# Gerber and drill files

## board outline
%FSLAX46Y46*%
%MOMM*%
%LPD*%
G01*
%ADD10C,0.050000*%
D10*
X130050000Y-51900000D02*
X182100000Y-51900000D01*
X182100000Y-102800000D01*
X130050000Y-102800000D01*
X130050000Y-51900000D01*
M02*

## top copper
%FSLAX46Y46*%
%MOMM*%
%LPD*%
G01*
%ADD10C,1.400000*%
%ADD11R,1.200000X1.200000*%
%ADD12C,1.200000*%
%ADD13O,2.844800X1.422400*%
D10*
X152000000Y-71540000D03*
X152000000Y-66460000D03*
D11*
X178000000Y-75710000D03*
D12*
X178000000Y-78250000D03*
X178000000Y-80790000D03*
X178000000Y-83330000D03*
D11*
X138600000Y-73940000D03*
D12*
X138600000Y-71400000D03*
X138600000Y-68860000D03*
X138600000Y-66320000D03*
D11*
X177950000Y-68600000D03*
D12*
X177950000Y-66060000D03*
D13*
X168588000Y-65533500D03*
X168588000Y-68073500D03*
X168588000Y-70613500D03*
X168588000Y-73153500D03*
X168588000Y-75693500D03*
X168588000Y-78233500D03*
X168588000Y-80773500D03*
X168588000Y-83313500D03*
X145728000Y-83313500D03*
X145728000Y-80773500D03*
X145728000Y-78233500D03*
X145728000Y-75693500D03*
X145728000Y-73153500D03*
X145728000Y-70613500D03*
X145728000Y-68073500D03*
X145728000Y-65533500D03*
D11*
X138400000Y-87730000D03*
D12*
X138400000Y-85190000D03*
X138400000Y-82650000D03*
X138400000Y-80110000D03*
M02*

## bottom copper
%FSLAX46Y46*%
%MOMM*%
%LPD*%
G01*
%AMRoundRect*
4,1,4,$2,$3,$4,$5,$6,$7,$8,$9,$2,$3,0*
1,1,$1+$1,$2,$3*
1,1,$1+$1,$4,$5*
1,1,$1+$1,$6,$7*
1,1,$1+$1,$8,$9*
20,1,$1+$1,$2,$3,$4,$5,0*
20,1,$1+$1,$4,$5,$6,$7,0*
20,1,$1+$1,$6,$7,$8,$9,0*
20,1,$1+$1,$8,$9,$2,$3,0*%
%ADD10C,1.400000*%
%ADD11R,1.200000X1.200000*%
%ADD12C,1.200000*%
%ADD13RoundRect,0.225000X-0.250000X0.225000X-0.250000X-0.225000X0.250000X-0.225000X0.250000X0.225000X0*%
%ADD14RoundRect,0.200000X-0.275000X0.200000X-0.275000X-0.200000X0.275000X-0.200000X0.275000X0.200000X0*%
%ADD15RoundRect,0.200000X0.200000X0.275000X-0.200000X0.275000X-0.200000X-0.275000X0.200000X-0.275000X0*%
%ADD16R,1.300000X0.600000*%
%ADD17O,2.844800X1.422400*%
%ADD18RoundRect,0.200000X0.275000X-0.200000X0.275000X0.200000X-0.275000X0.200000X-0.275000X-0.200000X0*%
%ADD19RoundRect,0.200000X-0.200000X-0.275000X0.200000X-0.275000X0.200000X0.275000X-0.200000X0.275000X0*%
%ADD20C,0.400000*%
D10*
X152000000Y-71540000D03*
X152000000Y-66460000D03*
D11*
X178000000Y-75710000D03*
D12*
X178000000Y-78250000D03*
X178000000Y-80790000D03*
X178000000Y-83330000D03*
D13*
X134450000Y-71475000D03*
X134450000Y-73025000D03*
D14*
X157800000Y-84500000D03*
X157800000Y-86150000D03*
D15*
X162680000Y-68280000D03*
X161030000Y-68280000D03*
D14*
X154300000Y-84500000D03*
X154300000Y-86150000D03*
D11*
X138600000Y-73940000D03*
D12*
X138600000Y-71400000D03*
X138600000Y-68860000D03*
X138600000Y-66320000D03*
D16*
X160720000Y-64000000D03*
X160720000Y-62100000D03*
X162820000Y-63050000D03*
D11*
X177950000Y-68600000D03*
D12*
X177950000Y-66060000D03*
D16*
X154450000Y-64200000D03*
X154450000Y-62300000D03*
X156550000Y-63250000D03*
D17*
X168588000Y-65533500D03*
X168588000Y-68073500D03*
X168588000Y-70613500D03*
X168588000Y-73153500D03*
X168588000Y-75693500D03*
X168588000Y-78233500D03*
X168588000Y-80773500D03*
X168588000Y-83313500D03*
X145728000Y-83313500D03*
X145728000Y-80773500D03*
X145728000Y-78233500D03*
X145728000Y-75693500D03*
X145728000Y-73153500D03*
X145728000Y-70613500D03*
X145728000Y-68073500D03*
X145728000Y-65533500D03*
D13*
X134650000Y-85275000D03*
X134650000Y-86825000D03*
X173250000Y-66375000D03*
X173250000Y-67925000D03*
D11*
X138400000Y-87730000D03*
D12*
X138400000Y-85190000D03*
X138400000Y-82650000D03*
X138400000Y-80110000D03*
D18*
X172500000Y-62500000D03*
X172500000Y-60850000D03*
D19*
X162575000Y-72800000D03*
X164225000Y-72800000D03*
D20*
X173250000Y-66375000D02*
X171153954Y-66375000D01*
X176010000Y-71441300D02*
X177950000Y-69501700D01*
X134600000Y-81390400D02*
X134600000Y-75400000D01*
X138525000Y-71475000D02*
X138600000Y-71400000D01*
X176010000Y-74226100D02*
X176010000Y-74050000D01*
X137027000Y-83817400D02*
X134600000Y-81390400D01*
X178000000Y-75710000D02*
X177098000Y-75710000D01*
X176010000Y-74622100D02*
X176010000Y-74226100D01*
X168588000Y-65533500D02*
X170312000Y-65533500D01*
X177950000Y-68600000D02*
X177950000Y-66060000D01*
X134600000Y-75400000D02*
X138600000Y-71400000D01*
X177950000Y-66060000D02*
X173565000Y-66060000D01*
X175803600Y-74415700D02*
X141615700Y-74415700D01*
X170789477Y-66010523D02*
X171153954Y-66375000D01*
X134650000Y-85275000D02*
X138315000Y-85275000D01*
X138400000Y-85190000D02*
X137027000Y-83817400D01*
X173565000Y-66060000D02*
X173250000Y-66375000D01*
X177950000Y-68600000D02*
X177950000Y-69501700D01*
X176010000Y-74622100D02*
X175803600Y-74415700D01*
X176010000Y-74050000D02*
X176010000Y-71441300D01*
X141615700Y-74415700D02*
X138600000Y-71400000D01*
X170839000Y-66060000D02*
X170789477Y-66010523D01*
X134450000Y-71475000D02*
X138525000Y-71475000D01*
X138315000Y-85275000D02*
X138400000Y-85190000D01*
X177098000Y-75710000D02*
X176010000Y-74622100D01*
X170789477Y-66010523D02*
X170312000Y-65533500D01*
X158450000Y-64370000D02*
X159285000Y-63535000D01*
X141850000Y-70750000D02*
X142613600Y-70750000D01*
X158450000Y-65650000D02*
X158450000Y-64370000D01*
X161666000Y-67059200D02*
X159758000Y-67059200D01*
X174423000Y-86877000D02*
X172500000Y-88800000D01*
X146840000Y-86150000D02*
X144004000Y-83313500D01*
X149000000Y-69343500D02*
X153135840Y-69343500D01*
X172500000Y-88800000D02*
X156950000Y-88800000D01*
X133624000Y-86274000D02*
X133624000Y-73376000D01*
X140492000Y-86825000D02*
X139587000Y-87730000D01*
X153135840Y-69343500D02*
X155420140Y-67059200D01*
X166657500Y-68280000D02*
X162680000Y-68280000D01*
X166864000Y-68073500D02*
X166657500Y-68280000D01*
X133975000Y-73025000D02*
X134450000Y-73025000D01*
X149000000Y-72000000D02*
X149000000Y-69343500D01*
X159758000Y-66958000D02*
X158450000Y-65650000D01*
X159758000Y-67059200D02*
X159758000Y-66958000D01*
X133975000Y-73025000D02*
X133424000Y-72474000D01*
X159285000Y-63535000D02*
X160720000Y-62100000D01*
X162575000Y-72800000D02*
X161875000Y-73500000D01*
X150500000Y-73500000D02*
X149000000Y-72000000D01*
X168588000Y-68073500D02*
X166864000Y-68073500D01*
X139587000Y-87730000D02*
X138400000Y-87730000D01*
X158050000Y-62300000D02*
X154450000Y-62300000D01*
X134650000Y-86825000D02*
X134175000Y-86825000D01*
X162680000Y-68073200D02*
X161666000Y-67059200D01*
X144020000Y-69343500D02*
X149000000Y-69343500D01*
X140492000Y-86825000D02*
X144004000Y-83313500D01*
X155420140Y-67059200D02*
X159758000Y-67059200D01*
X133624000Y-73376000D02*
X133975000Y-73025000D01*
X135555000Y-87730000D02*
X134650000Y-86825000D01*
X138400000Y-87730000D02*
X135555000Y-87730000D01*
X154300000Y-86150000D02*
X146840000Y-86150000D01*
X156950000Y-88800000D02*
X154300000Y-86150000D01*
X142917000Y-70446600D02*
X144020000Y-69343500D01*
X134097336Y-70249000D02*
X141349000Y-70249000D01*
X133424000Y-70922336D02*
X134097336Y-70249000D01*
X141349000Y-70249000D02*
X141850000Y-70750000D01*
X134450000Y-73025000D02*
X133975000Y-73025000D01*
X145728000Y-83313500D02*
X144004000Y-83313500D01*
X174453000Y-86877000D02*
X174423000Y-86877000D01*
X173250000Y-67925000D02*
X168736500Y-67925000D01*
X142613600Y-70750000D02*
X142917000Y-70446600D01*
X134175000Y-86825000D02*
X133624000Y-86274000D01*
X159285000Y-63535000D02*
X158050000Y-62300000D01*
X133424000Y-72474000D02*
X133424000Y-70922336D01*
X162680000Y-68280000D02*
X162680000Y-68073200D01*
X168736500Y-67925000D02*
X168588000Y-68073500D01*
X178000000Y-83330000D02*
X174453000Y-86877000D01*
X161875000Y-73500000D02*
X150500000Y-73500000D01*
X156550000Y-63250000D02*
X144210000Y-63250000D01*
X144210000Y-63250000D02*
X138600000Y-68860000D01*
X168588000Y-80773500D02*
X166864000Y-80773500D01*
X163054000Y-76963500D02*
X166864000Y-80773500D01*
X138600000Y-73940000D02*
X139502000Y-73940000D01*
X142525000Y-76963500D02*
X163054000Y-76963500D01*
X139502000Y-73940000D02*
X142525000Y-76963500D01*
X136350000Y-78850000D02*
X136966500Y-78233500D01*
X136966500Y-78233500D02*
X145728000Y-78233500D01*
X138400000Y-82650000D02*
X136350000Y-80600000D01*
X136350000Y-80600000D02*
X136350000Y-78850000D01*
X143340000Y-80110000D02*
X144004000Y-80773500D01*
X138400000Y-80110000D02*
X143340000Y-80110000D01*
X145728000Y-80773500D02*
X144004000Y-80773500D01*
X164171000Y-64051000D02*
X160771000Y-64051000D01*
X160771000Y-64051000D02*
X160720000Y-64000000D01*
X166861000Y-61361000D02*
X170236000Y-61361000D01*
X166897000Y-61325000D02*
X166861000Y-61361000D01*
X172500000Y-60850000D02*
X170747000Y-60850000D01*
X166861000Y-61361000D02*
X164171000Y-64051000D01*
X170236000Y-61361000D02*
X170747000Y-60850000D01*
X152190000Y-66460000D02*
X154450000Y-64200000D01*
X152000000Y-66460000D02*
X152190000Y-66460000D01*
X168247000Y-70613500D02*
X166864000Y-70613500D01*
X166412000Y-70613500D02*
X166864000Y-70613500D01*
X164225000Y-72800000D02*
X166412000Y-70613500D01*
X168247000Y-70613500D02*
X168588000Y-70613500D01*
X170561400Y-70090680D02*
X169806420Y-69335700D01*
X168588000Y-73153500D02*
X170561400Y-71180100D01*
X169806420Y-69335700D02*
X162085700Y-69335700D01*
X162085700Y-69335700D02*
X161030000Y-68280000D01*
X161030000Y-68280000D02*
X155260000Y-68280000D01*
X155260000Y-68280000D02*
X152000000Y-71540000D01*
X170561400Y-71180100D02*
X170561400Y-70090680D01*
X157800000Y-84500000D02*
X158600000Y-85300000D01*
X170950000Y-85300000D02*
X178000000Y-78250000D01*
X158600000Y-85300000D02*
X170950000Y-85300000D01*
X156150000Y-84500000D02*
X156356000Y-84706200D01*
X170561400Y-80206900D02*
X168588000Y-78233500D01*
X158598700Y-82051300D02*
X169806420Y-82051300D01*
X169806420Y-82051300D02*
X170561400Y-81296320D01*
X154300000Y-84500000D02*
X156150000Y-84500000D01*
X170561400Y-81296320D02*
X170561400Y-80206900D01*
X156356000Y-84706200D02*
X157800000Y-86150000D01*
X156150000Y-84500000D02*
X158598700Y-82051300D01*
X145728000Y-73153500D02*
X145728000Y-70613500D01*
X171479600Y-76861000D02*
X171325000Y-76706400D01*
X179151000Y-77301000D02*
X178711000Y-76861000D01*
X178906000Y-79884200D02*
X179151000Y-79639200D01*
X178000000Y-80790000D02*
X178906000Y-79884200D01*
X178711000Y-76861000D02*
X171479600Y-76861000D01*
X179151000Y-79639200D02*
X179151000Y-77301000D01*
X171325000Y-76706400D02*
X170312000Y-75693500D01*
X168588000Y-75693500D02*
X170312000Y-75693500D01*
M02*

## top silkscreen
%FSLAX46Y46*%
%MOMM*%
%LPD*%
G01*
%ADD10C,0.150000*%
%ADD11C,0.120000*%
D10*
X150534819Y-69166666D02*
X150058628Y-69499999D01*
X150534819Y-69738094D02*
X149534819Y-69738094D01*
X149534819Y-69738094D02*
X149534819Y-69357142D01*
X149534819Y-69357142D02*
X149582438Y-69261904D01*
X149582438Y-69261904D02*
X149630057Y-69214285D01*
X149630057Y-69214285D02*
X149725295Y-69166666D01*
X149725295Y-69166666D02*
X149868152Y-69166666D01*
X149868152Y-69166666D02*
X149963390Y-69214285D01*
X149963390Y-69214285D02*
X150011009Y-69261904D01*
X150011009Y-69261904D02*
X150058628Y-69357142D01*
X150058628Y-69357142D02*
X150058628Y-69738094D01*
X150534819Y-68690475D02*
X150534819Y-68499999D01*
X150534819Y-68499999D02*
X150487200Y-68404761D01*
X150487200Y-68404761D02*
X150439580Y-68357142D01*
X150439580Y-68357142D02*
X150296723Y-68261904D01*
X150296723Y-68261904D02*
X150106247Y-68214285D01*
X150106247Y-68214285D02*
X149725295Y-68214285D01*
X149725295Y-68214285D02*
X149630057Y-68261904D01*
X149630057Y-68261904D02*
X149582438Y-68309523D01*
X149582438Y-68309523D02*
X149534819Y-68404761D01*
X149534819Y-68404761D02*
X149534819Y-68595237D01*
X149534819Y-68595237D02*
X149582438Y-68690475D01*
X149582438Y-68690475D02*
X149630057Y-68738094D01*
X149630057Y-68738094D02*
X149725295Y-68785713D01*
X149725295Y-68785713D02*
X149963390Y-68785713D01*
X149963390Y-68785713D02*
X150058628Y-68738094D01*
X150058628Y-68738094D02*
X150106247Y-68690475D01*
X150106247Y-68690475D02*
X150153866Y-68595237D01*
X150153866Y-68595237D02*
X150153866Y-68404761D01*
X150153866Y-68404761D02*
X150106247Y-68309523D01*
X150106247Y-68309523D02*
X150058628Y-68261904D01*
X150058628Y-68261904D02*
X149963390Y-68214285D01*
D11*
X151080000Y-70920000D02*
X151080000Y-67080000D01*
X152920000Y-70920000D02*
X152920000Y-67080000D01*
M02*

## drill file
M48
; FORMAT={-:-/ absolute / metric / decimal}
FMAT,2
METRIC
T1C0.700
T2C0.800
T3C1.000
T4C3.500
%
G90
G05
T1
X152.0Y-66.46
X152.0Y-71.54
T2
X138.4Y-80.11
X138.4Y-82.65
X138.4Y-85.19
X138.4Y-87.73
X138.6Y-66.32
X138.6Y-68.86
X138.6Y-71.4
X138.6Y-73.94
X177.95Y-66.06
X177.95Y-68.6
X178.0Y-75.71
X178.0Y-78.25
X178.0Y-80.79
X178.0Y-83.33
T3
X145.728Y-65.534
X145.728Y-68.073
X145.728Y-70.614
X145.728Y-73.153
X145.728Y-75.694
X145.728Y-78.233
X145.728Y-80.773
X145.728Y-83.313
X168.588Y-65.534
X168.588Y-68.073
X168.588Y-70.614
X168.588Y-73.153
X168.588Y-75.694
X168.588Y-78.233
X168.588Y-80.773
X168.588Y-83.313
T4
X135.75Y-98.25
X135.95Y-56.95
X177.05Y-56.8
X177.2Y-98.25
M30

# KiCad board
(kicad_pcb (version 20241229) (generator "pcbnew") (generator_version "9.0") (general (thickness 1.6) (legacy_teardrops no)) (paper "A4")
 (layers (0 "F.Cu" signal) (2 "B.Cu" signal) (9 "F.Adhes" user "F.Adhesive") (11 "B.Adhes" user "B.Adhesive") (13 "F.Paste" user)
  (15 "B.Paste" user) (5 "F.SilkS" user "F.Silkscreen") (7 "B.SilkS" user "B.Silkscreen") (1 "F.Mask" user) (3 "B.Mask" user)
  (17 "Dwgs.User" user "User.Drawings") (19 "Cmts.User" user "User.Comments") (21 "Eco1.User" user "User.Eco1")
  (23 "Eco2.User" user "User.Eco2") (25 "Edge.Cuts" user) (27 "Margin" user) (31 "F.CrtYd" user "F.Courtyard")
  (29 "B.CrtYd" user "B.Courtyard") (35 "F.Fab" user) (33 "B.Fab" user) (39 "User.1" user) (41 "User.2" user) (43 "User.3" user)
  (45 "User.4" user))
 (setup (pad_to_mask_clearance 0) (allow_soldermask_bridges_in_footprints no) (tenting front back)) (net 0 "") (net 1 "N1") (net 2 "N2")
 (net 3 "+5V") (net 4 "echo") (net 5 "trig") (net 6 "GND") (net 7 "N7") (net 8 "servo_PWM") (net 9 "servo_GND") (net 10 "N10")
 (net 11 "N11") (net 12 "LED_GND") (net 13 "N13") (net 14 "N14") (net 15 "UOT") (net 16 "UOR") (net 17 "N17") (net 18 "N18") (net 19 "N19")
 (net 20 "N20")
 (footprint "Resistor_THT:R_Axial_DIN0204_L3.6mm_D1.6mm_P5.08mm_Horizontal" (layer "F.Cu") (at 152 71.54 90)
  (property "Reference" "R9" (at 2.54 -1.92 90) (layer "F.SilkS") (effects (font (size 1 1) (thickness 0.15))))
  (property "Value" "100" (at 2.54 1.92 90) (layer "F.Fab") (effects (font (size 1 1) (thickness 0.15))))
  (fp_line (start 0.62 -0.92) (end 4.46 -0.92) (stroke (width 0.12) (type solid)) (layer "F.SilkS"))
  (fp_line (start 0.62 0.92) (end 4.46 0.92) (stroke (width 0.12) (type solid)) (layer "F.SilkS"))
  (pad "1" thru_hole circle (at 0 0 90) (size 1.4 1.4) (drill 0.7) (layers "*.Cu" "*.Mask") (remove_unused_layers no) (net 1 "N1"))
  (pad "2" thru_hole circle (at 5.08 0 90) (size 1.4 1.4) (drill 0.7) (layers "*.Cu" "*.Mask") (remove_unused_layers no) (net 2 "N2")))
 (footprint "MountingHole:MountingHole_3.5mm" (layer "B.Cu") (at 135.75 98.25 180)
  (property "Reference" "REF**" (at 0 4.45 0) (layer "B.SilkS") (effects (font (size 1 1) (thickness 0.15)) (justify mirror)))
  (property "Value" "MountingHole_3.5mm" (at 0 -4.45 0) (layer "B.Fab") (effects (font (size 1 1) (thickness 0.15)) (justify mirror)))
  (pad "" np_thru_hole circle (at 0 0 180) (size 3.5 3.5) (drill 3.5) (layers "*.Cu" "*.Mask")))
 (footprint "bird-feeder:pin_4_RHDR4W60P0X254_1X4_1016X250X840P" (layer "B.Cu") (at 178 75.71 -90)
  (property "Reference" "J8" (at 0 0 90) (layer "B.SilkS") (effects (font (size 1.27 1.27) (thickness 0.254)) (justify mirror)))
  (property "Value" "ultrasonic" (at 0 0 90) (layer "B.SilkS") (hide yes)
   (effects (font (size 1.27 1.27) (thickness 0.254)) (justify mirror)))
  (pad "1" thru_hole rect (at 0 0 270) (size 1.2 1.2) (drill 0.8) (layers "*.Cu" "*.Mask") (remove_unused_layers no) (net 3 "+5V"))
  (pad "2" thru_hole circle (at 2.54 0 270) (size 1.2 1.2) (drill 0.8) (layers "*.Cu" "*.Mask") (remove_unused_layers no) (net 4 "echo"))
  (pad "3" thru_hole circle (at 5.08 0 270) (size 1.2 1.2) (drill 0.8) (layers "*.Cu" "*.Mask") (remove_unused_layers no) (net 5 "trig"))
  (pad "4" thru_hole circle (at 7.62 0 270) (size 1.2 1.2) (drill 0.8) (layers "*.Cu" "*.Mask") (remove_unused_layers no) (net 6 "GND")))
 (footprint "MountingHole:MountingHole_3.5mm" (layer "B.Cu") (at 135.95 56.95 180)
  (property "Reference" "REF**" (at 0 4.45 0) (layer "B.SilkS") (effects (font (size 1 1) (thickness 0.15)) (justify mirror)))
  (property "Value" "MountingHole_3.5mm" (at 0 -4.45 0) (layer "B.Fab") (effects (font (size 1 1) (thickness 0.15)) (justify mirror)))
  (pad "" np_thru_hole circle (at 0 0 180) (size 3.5 3.5) (drill 3.5) (layers "*.Cu" "*.Mask")))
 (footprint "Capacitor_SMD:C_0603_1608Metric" (layer "B.Cu") (at 134.45 72.25 -90)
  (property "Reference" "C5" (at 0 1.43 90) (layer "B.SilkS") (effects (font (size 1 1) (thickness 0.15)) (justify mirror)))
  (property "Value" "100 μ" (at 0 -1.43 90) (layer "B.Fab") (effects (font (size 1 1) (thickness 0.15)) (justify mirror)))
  (pad "1" smd roundrect (at -0.775 0 270) (size 0.9 0.95) (layers "B.Cu" "B.Mask" "B.Paste") (roundrect_rratio 0.25) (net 3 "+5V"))
  (pad "2" smd roundrect (at 0.775 0 270) (size 0.9 0.95) (layers "B.Cu" "B.Mask" "B.Paste") (roundrect_rratio 0.25) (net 6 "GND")))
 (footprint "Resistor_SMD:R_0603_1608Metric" (layer "B.Cu") (at 157.8 85.325 -90)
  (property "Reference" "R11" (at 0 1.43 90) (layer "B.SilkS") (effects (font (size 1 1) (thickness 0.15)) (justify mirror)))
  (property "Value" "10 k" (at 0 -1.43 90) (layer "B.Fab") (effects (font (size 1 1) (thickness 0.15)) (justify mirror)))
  (pad "1" smd roundrect (at -0.825 0 270) (size 0.8 0.95) (layers "B.Cu" "B.Mask" "B.Paste") (roundrect_rratio 0.25) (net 4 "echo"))
  (pad "2" smd roundrect (at 0.825 0 270) (size 0.8 0.95) (layers "B.Cu" "B.Mask" "B.Paste") (roundrect_rratio 0.25) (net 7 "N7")))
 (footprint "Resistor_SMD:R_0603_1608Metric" (layer "B.Cu") (at 161.855 68.28 180)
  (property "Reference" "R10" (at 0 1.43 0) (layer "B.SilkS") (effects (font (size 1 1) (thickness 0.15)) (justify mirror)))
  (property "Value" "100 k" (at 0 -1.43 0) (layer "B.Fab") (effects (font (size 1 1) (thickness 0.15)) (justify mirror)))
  (pad "1" smd roundrect (at -0.825 0 180) (size 0.8 0.95) (layers "B.Cu" "B.Mask" "B.Paste") (roundrect_rratio 0.25) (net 6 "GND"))
  (pad "2" smd roundrect (at 0.825 0 180) (size 0.8 0.95) (layers "B.Cu" "B.Mask" "B.Paste") (roundrect_rratio 0.25) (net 1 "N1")))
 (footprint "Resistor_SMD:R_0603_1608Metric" (layer "B.Cu") (at 154.3 85.325 -90)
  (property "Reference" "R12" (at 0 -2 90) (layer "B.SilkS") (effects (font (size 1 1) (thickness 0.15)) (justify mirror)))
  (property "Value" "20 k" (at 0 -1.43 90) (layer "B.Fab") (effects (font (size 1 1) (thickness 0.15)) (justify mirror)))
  (pad "1" smd roundrect (at -0.825 0 270) (size 0.8 0.95) (layers "B.Cu" "B.Mask" "B.Paste") (roundrect_rratio 0.25) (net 7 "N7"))
  (pad "2" smd roundrect (at 0.825 0 270) (size 0.8 0.95) (layers "B.Cu" "B.Mask" "B.Paste") (roundrect_rratio 0.25) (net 6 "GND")))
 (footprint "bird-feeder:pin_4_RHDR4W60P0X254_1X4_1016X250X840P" (layer "B.Cu") (at 138.6 73.94 90)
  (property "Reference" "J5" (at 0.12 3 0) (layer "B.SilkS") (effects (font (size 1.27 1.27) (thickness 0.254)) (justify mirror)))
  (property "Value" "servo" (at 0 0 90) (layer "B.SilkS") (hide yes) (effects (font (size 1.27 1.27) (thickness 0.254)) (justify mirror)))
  (pad "1" thru_hole rect (at 0 0 90) (size 1.2 1.2) (drill 0.8) (layers "*.Cu" "*.Mask") (remove_unused_layers no) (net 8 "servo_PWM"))
  (pad "2" thru_hole circle (at 2.54 0 90) (size 1.2 1.2) (drill 0.8) (layers "*.Cu" "*.Mask") (remove_unused_layers no) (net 3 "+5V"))
  (pad "3" thru_hole circle (at 5.08 0 90) (size 1.2 1.2) (drill 0.8) (layers "*.Cu" "*.Mask") (remove_unused_layers no) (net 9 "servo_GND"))
  (pad "4" thru_hole circle (at 7.62 0 90) (size 1.2 1.2) (drill 0.8) (layers "*.Cu" "*.Mask") (remove_unused_layers no) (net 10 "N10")))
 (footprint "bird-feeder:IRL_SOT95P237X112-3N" (layer "B.Cu") (at 161.77 63.05)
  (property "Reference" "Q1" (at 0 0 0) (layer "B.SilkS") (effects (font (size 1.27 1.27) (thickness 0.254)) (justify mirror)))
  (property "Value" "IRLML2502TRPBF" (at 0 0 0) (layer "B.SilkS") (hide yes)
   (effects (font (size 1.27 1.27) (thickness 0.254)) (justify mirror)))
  (pad "1" smd rect (at -1.05 0.95 270) (size 0.6 1.3) (layers "B.Cu" "B.Mask" "B.Paste") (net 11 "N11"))
  (pad "2" smd rect (at -1.05 -0.95 270) (size 0.6 1.3) (layers "B.Cu" "B.Mask" "B.Paste") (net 6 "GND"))
  (pad "3" smd rect (at 1.05 0 270) (size 0.6 1.3) (layers "B.Cu" "B.Mask" "B.Paste") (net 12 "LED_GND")))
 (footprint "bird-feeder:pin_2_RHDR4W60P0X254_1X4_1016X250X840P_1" (layer "B.Cu") (at 177.95 68.6 90)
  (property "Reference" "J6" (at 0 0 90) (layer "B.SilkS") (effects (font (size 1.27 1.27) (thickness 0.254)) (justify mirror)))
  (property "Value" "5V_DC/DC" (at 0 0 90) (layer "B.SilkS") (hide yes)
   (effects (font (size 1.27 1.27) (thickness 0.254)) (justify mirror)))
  (pad "1" thru_hole rect (at 0 0 90) (size 1.2 1.2) (drill 0.8) (layers "*.Cu" "*.Mask") (remove_unused_layers no) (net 3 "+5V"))
  (pad "2" thru_hole circle (at 2.54 0 90) (size 1.2 1.2) (drill 0.8) (layers "*.Cu" "*.Mask") (remove_unused_layers no) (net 3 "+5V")))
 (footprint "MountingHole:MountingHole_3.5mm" (layer "B.Cu") (at 177.2 98.25 180)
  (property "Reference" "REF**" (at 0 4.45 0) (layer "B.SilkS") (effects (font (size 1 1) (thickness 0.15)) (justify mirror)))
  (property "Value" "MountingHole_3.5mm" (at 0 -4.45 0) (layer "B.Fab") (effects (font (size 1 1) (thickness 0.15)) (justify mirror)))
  (pad "" np_thru_hole circle (at 0 0 180) (size 3.5 3.5) (drill 3.5) (layers "*.Cu" "*.Mask")))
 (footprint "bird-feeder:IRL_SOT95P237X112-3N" (layer "B.Cu") (at 155.5 63.25)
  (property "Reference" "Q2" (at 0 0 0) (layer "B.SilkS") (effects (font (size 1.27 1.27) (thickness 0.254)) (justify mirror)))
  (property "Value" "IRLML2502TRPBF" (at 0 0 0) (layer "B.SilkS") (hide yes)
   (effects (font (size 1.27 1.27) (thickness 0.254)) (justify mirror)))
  (pad "1" smd rect (at -1.05 0.95 270) (size 0.6 1.3) (layers "B.Cu" "B.Mask" "B.Paste") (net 2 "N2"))
  (pad "2" smd rect (at -1.05 -0.95 270) (size 0.6 1.3) (layers "B.Cu" "B.Mask" "B.Paste") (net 6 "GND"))
  (pad "3" smd rect (at 1.05 0 270) (size 0.6 1.3) (layers "B.Cu" "B.Mask" "B.Paste") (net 9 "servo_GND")))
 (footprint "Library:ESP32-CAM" (layer "B.Cu") (at 157.158 75.6935 180)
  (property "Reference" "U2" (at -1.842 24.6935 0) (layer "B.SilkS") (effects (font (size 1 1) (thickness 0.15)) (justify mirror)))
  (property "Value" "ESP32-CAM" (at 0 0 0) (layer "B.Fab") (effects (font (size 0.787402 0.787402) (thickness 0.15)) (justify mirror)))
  (pad "P$1" thru_hole oval (at -11.43 10.16 180) (size 2.8448 1.4224) (drill 1) (layers "*.Cu" "*.Mask") (remove_unused_layers no)
   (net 3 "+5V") (solder_mask_margin 0.102))
  (pad "P$2" thru_hole oval (at -11.43 7.62 180) (size 2.8448 1.4224) (drill 1) (layers "*.Cu" "*.Mask") (remove_unused_layers no)
   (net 6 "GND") (solder_mask_margin 0.102))
  (pad "P$3" thru_hole oval (at -11.43 5.08 180) (size 2.8448 1.4224) (drill 1) (layers "*.Cu" "*.Mask") (remove_unused_layers no)
   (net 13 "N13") (solder_mask_margin 0.102))
  (pad "P$4" thru_hole oval (at -11.43 2.54 180) (size 2.8448 1.4224) (drill 1) (layers "*.Cu" "*.Mask") (remove_unused_layers no)
   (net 1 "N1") (solder_mask_margin 0.102))
  (pad "P$5" thru_hole oval (at -11.43 0 180) (size 2.8448 1.4224) (drill 1) (layers "*.Cu" "*.Mask") (remove_unused_layers no)
   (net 5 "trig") (solder_mask_margin 0.102))
  (pad "P$6" thru_hole oval (at -11.43 -2.54 180) (size 2.8448 1.4224) (drill 1) (layers "*.Cu" "*.Mask") (remove_unused_layers no)
   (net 7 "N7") (solder_mask_margin 0.102))
  (pad "P$7" thru_hole oval (at -11.43 -5.08 180) (size 2.8448 1.4224) (drill 1) (layers "*.Cu" "*.Mask") (remove_unused_layers no)
   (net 8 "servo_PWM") (solder_mask_margin 0.102))
  (pad "P$8" thru_hole oval (at -11.43 -7.62 180) (size 2.8448 1.4224) (drill 1) (layers "*.Cu" "*.Mask") (remove_unused_layers no)
   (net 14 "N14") (solder_mask_margin 0.102))
  (pad "P$9" thru_hole oval (at 11.43 -7.62 180) (size 2.8448 1.4224) (drill 1) (layers "*.Cu" "*.Mask") (remove_unused_layers no)
   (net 6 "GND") (solder_mask_margin 0.102))
  (pad "P$10" thru_hole oval (at 11.43 -5.08 180) (size 2.8448 1.4224) (drill 1) (layers "*.Cu" "*.Mask") (remove_unused_layers no)
   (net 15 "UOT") (solder_mask_margin 0.102))
  (pad "P$11" thru_hole oval (at 11.43 -2.54 180) (size 2.8448 1.4224) (drill 1) (layers "*.Cu" "*.Mask") (remove_unused_layers no)
   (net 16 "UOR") (solder_mask_margin 0.102))
  (pad "P$12" thru_hole oval (at 11.43 0 180) (size 2.8448 1.4224) (drill 1) (layers "*.Cu" "*.Mask") (remove_unused_layers no)
   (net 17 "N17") (solder_mask_margin 0.102))
  (pad "P$13" thru_hole oval (at 11.43 2.54 180) (size 2.8448 1.4224) (drill 1) (layers "*.Cu" "*.Mask") (remove_unused_layers no)
   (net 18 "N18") (solder_mask_margin 0.102))
  (pad "P$14" thru_hole oval (at 11.43 5.08 180) (size 2.8448 1.4224) (drill 1) (layers "*.Cu" "*.Mask") (remove_unused_layers no)
   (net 18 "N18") (solder_mask_margin 0.102))
  (pad "P$15" thru_hole oval (at 11.43 7.62 180) (size 2.8448 1.4224) (drill 1) (layers "*.Cu" "*.Mask") (remove_unused_layers no)
   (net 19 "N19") (solder_mask_margin 0.102))
  (pad "P$16" thru_hole oval (at 11.43 10.16 180) (size 2.8448 1.4224) (drill 1) (layers "*.Cu" "*.Mask") (remove_unused_layers no)
   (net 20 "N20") (solder_mask_margin 0.102)))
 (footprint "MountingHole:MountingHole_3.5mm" (layer "B.Cu") (at 177.05 56.8 180)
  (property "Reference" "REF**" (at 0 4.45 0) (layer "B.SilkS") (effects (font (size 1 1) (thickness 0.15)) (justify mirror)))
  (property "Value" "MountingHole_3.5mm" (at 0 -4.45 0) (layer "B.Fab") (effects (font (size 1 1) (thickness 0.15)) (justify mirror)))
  (pad "" np_thru_hole circle (at 0 0 180) (size 3.5 3.5) (drill 3.5) (layers "*.Cu" "*.Mask")))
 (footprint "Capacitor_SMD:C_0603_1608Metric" (layer "B.Cu") (at 134.65 86.05 -90)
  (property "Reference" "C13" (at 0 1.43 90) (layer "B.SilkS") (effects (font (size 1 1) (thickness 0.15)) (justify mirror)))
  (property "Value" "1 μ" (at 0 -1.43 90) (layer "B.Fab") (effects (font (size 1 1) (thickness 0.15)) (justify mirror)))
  (pad "1" smd roundrect (at -0.775 0 270) (size 0.9 0.95) (layers "B.Cu" "B.Mask" "B.Paste") (roundrect_rratio 0.25) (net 3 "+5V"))
  (pad "2" smd roundrect (at 0.775 0 270) (size 0.9 0.95) (layers "B.Cu" "B.Mask" "B.Paste") (roundrect_rratio 0.25) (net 6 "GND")))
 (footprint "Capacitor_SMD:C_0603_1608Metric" (layer "B.Cu") (at 173.25 67.15 -90)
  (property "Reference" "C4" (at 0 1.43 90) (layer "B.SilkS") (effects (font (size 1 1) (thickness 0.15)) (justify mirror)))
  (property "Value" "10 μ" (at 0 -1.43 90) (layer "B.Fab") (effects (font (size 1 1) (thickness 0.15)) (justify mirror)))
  (pad "1" smd roundrect (at -0.775 0 270) (size 0.9 0.95) (layers "B.Cu" "B.Mask" "B.Paste") (roundrect_rratio 0.25) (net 3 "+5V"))
  (pad "2" smd roundrect (at 0.775 0 270) (size 0.9 0.95) (layers "B.Cu" "B.Mask" "B.Paste") (roundrect_rratio 0.25) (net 6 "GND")))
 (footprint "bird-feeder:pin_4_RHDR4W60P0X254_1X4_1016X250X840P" (layer "B.Cu") (at 138.4 87.73 90)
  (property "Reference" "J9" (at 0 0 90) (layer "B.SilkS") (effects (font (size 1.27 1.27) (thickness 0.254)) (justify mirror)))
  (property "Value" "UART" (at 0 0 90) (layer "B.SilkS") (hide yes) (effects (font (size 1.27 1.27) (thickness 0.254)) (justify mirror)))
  (pad "1" thru_hole rect (at 0 0 90) (size 1.2 1.2) (drill 0.8) (layers "*.Cu" "*.Mask") (remove_unused_layers no) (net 6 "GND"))
  (pad "2" thru_hole circle (at 2.54 0 90) (size 1.2 1.2) (drill 0.8) (layers "*.Cu" "*.Mask") (remove_unused_layers no) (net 3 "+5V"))
  (pad "3" thru_hole circle (at 5.08 0 90) (size 1.2 1.2) (drill 0.8) (layers "*.Cu" "*.Mask") (remove_unused_layers no) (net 16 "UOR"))
  (pad "4" thru_hole circle (at 7.62 0 90) (size 1.2 1.2) (drill 0.8) (layers "*.Cu" "*.Mask") (remove_unused_layers no) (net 15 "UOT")))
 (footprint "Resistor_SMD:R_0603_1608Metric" (layer "B.Cu") (at 172.5 61.675 90)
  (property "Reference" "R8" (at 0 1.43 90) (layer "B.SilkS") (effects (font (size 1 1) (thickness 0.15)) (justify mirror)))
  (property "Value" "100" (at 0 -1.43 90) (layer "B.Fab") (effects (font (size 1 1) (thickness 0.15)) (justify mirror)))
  (pad "1" smd roundrect (at -0.825 0 90) (size 0.8 0.95) (layers "B.Cu" "B.Mask" "B.Paste") (roundrect_rratio 0.25) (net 13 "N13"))
  (pad "2" smd roundrect (at 0.825 0 90) (size 0.8 0.95) (layers "B.Cu" "B.Mask" "B.Paste") (roundrect_rratio 0.25) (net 11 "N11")))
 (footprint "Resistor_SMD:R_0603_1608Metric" (layer "B.Cu") (at 163.4 72.8)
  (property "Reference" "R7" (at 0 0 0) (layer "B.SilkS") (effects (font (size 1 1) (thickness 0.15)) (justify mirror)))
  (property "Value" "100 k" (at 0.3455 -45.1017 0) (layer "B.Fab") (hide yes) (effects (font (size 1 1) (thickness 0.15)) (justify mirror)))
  (pad "1" smd roundrect (at -0.825 0) (size 0.8 0.95) (layers "B.Cu" "B.Mask" "B.Paste") (roundrect_rratio 0.25) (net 6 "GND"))
  (pad "2" smd roundrect (at 0.825 0) (size 0.8 0.95) (layers "B.Cu" "B.Mask" "B.Paste") (roundrect_rratio 0.25) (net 13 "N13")))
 (gr_rect (start 130.05 51.9) (end 182.1 102.8) (stroke (width 0.05) (type default)) (fill no) (layer "Edge.Cuts"))
 (segment (start 173.25 66.375) (end 171.153954 66.375) (width 0.4) (layer "B.Cu") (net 3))
 (segment (start 176.01 71.4413) (end 177.95 69.5017) (width 0.4) (layer "B.Cu") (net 3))
 (segment (start 134.6 81.3904) (end 134.6 75.4) (width 0.4) (layer "B.Cu") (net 3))
 (segment (start 138.525 71.475) (end 138.6 71.4) (width 0.4) (layer "B.Cu") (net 3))
 (segment (start 176.01 74.2261) (end 176.01 74.05) (width 0.4) (layer "B.Cu") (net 3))
 (segment (start 137.027 83.8174) (end 134.6 81.3904) (width 0.4) (layer "B.Cu") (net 3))
 (segment (start 178 75.71) (end 177.098 75.71) (width 0.4) (layer "B.Cu") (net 3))
 (segment (start 176.01 74.6221) (end 176.01 74.2261) (width 0.4) (layer "B.Cu") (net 3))
 (segment (start 168.588 65.5335) (end 170.312 65.5335) (width 0.4) (layer "B.Cu") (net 3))
 (segment (start 177.95 68.6) (end 177.95 66.06) (width 0.4) (layer "B.Cu") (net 3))
 (segment (start 134.6 75.4) (end 138.6 71.4) (width 0.4) (layer "B.Cu") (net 3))
 (segment (start 177.95 66.06) (end 173.565 66.06) (width 0.4) (layer "B.Cu") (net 3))
 (segment (start 175.8036 74.4157) (end 141.6157 74.4157) (width 0.4) (layer "B.Cu") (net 3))
 (segment (start 170.789477 66.010523) (end 171.153954 66.375) (width 0.4) (layer "B.Cu") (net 3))
 (segment (start 134.65 85.275) (end 138.315 85.275) (width 0.4) (layer "B.Cu") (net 3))
 (segment (start 138.4 85.19) (end 137.027 83.8174) (width 0.4) (layer "B.Cu") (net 3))
 (segment (start 173.565 66.06) (end 173.25 66.375) (width 0.4) (layer "B.Cu") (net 3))
 (segment (start 177.95 68.6) (end 177.95 69.5017) (width 0.4) (layer "B.Cu") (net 3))
 (segment (start 176.01 74.6221) (end 175.8036 74.4157) (width 0.4) (layer "B.Cu") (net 3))
 (segment (start 176.01 74.05) (end 176.01 71.4413) (width 0.4) (layer "B.Cu") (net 3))
 (segment (start 141.6157 74.4157) (end 138.6 71.4) (width 0.4) (layer "B.Cu") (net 3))
 (segment (start 170.839 66.06) (end 170.789477 66.010523) (width 0.4) (layer "B.Cu") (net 3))
 (segment (start 134.45 71.475) (end 138.525 71.475) (width 0.4) (layer "B.Cu") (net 3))
 (segment (start 138.315 85.275) (end 138.4 85.19) (width 0.4) (layer "B.Cu") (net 3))
 (segment (start 177.098 75.71) (end 176.01 74.6221) (width 0.4) (layer "B.Cu") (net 3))
 (segment (start 170.789477 66.010523) (end 170.312 65.5335) (width 0.4) (layer "B.Cu") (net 3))
 (segment (start 158.45 64.37) (end 159.285 63.535) (width 0.4) (layer "B.Cu") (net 6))
 (segment (start 141.85 70.75) (end 142.6136 70.75) (width 0.4) (layer "B.Cu") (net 6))
 (segment (start 158.45 65.65) (end 158.45 64.37) (width 0.4) (layer "B.Cu") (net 6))
 (segment (start 161.666 67.0592) (end 159.758 67.0592) (width 0.4) (layer "B.Cu") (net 6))
 (segment (start 174.423 86.877) (end 172.5 88.8) (width 0.4) (layer "B.Cu") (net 6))
 (segment (start 146.84 86.15) (end 144.004 83.3135) (width 0.4) (layer "B.Cu") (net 6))
 (segment (start 149 69.3435) (end 153.13584 69.3435) (width 0.4) (layer "B.Cu") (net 6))
 (segment (start 172.5 88.8) (end 156.95 88.8) (width 0.4) (layer "B.Cu") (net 6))
 (segment (start 133.624 86.274) (end 133.624 73.376) (width 0.4) (layer "B.Cu") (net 6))
 (segment (start 140.492 86.825) (end 139.587 87.73) (width 0.4) (layer "B.Cu") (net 6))
 (segment (start 153.13584 69.3435) (end 155.42014 67.0592) (width 0.4) (layer "B.Cu") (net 6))
 (segment (start 166.6575 68.28) (end 162.68 68.28) (width 0.4) (layer "B.Cu") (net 6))
 (segment (start 166.864 68.0735) (end 166.6575 68.28) (width 0.4) (layer "B.Cu") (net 6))
 (segment (start 133.975 73.025) (end 134.45 73.025) (width 0.4) (layer "B.Cu") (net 6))
 (segment (start 149 72) (end 149 69.3435) (width 0.4) (layer "B.Cu") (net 6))
 (segment (start 159.758 66.958) (end 158.45 65.65) (width 0.4) (layer "B.Cu") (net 6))
 (segment (start 159.758 67.0592) (end 159.758 66.958) (width 0.4) (layer "B.Cu") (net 6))
 (segment (start 133.975 73.025) (end 133.424 72.474) (width 0.4) (layer "B.Cu") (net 6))
 (segment (start 159.285 63.535) (end 160.72 62.1) (width 0.4) (layer "B.Cu") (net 6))
 (segment (start 162.575 72.8) (end 161.875 73.5) (width 0.4) (layer "B.Cu") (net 6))
 (segment (start 150.5 73.5) (end 149 72) (width 0.4) (layer "B.Cu") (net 6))
 (segment (start 168.588 68.0735) (end 166.864 68.0735) (width 0.4) (layer "B.Cu") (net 6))
 (segment (start 139.587 87.73) (end 138.4 87.73) (width 0.4) (layer "B.Cu") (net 6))
 (segment (start 158.05 62.3) (end 154.45 62.3) (width 0.4) (layer "B.Cu") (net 6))
 (segment (start 134.65 86.825) (end 134.175 86.825) (width 0.4) (layer "B.Cu") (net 6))
 (segment (start 162.68 68.0732) (end 161.666 67.0592) (width 0.4) (layer "B.Cu") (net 6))
 (segment (start 144.02 69.3435) (end 149 69.3435) (width 0.4) (layer "B.Cu") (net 6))
 (segment (start 140.492 86.825) (end 144.004 83.3135) (width 0.4) (layer "B.Cu") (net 6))
 (segment (start 155.42014 67.0592) (end 159.758 67.0592) (width 0.4) (layer "B.Cu") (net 6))
 (segment (start 133.624 73.376) (end 133.975 73.025) (width 0.4) (layer "B.Cu") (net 6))
 (segment (start 135.555 87.73) (end 134.65 86.825) (width 0.4) (layer "B.Cu") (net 6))
 (segment (start 138.4 87.73) (end 135.555 87.73) (width 0.4) (layer "B.Cu") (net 6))
 (segment (start 154.3 86.15) (end 146.84 86.15) (width 0.4) (layer "B.Cu") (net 6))
 (segment (start 156.95 88.8) (end 154.3 86.15) (width 0.4) (layer "B.Cu") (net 6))
 (segment (start 142.917 70.4466) (end 144.02 69.3435) (width 0.4) (layer "B.Cu") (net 6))
 (segment (start 134.097336 70.249) (end 141.349 70.249) (width 0.4) (layer "B.Cu") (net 6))
 (segment (start 133.424 70.922336) (end 134.097336 70.249) (width 0.4) (layer "B.Cu") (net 6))
 (segment (start 141.349 70.249) (end 141.85 70.75) (width 0.4) (layer "B.Cu") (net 6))
 (segment (start 134.45 73.025) (end 133.975 73.025) (width 0.4) (layer "B.Cu") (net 6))
 (segment (start 145.728 83.3135) (end 144.004 83.3135) (width 0.4) (layer "B.Cu") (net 6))
 (segment (start 174.453 86.877) (end 174.423 86.877) (width 0.4) (layer "B.Cu") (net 6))
 (segment (start 173.25 67.925) (end 168.7365 67.925) (width 0.4) (layer "B.Cu") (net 6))
 (segment (start 142.6136 70.75) (end 142.917 70.4466) (width 0.4) (layer "B.Cu") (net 6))
 (segment (start 134.175 86.825) (end 133.624 86.274) (width 0.4) (layer "B.Cu") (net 6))
 (segment (start 159.285 63.535) (end 158.05 62.3) (width 0.4) (layer "B.Cu") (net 6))
 (segment (start 133.424 72.474) (end 133.424 70.922336) (width 0.4) (layer "B.Cu") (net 6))
 (segment (start 162.68 68.28) (end 162.68 68.0732) (width 0.4) (layer "B.Cu") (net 6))
 (segment (start 168.7365 67.925) (end 168.588 68.0735) (width 0.4) (layer "B.Cu") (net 6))
 (segment (start 178 83.33) (end 174.453 86.877) (width 0.4) (layer "B.Cu") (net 6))
 (segment (start 161.875 73.5) (end 150.5 73.5) (width 0.4) (layer "B.Cu") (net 6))
 (segment (start 156.55 63.25) (end 144.21 63.25) (width 0.4) (layer "B.Cu") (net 9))
 (segment (start 144.21 63.25) (end 138.6 68.86) (width 0.4) (layer "B.Cu") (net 9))
 (segment (start 168.588 80.7735) (end 166.864 80.7735) (width 0.4) (layer "B.Cu") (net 8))
 (segment (start 163.054 76.9635) (end 166.864 80.7735) (width 0.4) (layer "B.Cu") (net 8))
 (segment (start 138.6 73.94) (end 139.502 73.94) (width 0.4) (layer "B.Cu") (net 8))
 (segment (start 142.525 76.9635) (end 163.054 76.9635) (width 0.4) (layer "B.Cu") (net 8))
 (segment (start 139.502 73.94) (end 142.525 76.9635) (width 0.4) (layer "B.Cu") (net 8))
 (segment (start 136.35 78.85) (end 136.9665 78.2335) (width 0.4) (layer "B.Cu") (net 16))
 (segment (start 136.9665 78.2335) (end 145.728 78.2335) (width 0.4) (layer "B.Cu") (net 16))
 (segment (start 138.4 82.65) (end 136.35 80.6) (width 0.4) (layer "B.Cu") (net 16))
 (segment (start 136.35 80.6) (end 136.35 78.85) (width 0.4) (layer "B.Cu") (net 16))
 (segment (start 143.34 80.11) (end 144.004 80.7735) (width 0.4) (layer "B.Cu") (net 15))
 (segment (start 138.4 80.11) (end 143.34 80.11) (width 0.4) (layer "B.Cu") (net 15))
 (segment (start 145.728 80.7735) (end 144.004 80.7735) (width 0.4) (layer "B.Cu") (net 15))
 (segment (start 164.171 64.051) (end 160.771 64.051) (width 0.4) (layer "B.Cu") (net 11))
 (segment (start 160.771 64.051) (end 160.72 64) (width 0.4) (layer "B.Cu") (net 11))
 (segment (start 166.861 61.361) (end 170.236 61.361) (width 0.4) (layer "B.Cu") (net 11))
 (segment (start 166.897 61.325) (end 166.861 61.361) (width 0.4) (layer "B.Cu") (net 11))
 (segment (start 172.5 60.85) (end 170.747 60.85) (width 0.4) (layer "B.Cu") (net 11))
 (segment (start 166.861 61.361) (end 164.171 64.051) (width 0.4) (layer "B.Cu") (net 11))
 (segment (start 170.236 61.361) (end 170.747 60.85) (width 0.4) (layer "B.Cu") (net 11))
 (segment (start 152.19 66.46) (end 154.45 64.2) (width 0.4) (layer "B.Cu") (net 2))
 (segment (start 152 66.46) (end 152.19 66.46) (width 0.4) (layer "B.Cu") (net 2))
 (segment (start 168.247 70.6135) (end 166.864 70.6135) (width 0.4) (layer "B.Cu") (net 13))
 (segment (start 166.412 70.6135) (end 166.864 70.6135) (width 0.4) (layer "B.Cu") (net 13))
 (segment (start 164.225 72.8) (end 166.412 70.6135) (width 0.4) (layer "B.Cu") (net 13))
 (segment (start 168.247 70.6135) (end 168.588 70.6135) (width 0.4) (layer "B.Cu") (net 13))
 (segment (start 170.5614 70.09068) (end 169.80642 69.3357) (width 0.4) (layer "B.Cu") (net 1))
 (segment (start 168.588 73.1535) (end 170.5614 71.1801) (width 0.4) (layer "B.Cu") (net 1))
 (segment (start 169.80642 69.3357) (end 162.0857 69.3357) (width 0.4) (layer "B.Cu") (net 1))
 (segment (start 162.0857 69.3357) (end 161.03 68.28) (width 0.4) (layer "B.Cu") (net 1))
 (segment (start 161.03 68.28) (end 155.26 68.28) (width 0.4) (layer "B.Cu") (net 1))
 (segment (start 155.26 68.28) (end 152 71.54) (width 0.4) (layer "B.Cu") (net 1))
 (segment (start 170.5614 71.1801) (end 170.5614 70.09068) (width 0.4) (layer "B.Cu") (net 1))
 (segment (start 157.8 84.5) (end 158.6 85.3) (width 0.4) (layer "B.Cu") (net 4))
 (segment (start 170.95 85.3) (end 178 78.25) (width 0.4) (layer "B.Cu") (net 4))
 (segment (start 158.6 85.3) (end 170.95 85.3) (width 0.4) (layer "B.Cu") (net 4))
 (segment (start 156.15 84.5) (end 156.356 84.7062) (width 0.4) (layer "B.Cu") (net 7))
 (segment (start 170.5614 80.2069) (end 168.588 78.2335) (width 0.4) (layer "B.Cu") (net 7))
 (segment (start 158.5987 82.0513) (end 169.80642 82.0513) (width 0.4) (layer "B.Cu") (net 7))
 (segment (start 169.80642 82.0513) (end 170.5614 81.29632) (width 0.4) (layer "B.Cu") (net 7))
 (segment (start 154.3 84.5) (end 156.15 84.5) (width 0.4) (layer "B.Cu") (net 7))
 (segment (start 170.5614 81.29632) (end 170.5614 80.2069) (width 0.4) (layer "B.Cu") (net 7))
 (segment (start 156.356 84.7062) (end 157.8 86.15) (width 0.4) (layer "B.Cu") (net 7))
 (segment (start 156.15 84.5) (end 158.5987 82.0513) (width 0.4) (layer "B.Cu") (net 7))
 (segment (start 145.728 73.1535) (end 145.728 70.6135) (width 0.4) (layer "B.Cu") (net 18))
 (segment (start 171.4796 76.861) (end 171.325 76.7064) (width 0.4) (layer "B.Cu") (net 5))
 (segment (start 179.151 77.301) (end 178.711 76.861) (width 0.4) (layer "B.Cu") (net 5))
 (segment (start 178.906 79.8842) (end 179.151 79.6392) (width 0.4) (layer "B.Cu") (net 5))
 (segment (start 178 80.79) (end 178.906 79.8842) (width 0.4) (layer "B.Cu") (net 5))
 (segment (start 178.711 76.861) (end 171.4796 76.861) (width 0.4) (layer "B.Cu") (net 5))
 (segment (start 179.151 79.6392) (end 179.151 77.301) (width 0.4) (layer "B.Cu") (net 5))
 (segment (start 171.325 76.7064) (end 170.312 75.6935) (width 0.4) (layer "B.Cu") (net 5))
 (segment (start 168.588 75.6935) (end 170.312 75.6935) (width 0.4) (layer "B.Cu") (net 5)))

